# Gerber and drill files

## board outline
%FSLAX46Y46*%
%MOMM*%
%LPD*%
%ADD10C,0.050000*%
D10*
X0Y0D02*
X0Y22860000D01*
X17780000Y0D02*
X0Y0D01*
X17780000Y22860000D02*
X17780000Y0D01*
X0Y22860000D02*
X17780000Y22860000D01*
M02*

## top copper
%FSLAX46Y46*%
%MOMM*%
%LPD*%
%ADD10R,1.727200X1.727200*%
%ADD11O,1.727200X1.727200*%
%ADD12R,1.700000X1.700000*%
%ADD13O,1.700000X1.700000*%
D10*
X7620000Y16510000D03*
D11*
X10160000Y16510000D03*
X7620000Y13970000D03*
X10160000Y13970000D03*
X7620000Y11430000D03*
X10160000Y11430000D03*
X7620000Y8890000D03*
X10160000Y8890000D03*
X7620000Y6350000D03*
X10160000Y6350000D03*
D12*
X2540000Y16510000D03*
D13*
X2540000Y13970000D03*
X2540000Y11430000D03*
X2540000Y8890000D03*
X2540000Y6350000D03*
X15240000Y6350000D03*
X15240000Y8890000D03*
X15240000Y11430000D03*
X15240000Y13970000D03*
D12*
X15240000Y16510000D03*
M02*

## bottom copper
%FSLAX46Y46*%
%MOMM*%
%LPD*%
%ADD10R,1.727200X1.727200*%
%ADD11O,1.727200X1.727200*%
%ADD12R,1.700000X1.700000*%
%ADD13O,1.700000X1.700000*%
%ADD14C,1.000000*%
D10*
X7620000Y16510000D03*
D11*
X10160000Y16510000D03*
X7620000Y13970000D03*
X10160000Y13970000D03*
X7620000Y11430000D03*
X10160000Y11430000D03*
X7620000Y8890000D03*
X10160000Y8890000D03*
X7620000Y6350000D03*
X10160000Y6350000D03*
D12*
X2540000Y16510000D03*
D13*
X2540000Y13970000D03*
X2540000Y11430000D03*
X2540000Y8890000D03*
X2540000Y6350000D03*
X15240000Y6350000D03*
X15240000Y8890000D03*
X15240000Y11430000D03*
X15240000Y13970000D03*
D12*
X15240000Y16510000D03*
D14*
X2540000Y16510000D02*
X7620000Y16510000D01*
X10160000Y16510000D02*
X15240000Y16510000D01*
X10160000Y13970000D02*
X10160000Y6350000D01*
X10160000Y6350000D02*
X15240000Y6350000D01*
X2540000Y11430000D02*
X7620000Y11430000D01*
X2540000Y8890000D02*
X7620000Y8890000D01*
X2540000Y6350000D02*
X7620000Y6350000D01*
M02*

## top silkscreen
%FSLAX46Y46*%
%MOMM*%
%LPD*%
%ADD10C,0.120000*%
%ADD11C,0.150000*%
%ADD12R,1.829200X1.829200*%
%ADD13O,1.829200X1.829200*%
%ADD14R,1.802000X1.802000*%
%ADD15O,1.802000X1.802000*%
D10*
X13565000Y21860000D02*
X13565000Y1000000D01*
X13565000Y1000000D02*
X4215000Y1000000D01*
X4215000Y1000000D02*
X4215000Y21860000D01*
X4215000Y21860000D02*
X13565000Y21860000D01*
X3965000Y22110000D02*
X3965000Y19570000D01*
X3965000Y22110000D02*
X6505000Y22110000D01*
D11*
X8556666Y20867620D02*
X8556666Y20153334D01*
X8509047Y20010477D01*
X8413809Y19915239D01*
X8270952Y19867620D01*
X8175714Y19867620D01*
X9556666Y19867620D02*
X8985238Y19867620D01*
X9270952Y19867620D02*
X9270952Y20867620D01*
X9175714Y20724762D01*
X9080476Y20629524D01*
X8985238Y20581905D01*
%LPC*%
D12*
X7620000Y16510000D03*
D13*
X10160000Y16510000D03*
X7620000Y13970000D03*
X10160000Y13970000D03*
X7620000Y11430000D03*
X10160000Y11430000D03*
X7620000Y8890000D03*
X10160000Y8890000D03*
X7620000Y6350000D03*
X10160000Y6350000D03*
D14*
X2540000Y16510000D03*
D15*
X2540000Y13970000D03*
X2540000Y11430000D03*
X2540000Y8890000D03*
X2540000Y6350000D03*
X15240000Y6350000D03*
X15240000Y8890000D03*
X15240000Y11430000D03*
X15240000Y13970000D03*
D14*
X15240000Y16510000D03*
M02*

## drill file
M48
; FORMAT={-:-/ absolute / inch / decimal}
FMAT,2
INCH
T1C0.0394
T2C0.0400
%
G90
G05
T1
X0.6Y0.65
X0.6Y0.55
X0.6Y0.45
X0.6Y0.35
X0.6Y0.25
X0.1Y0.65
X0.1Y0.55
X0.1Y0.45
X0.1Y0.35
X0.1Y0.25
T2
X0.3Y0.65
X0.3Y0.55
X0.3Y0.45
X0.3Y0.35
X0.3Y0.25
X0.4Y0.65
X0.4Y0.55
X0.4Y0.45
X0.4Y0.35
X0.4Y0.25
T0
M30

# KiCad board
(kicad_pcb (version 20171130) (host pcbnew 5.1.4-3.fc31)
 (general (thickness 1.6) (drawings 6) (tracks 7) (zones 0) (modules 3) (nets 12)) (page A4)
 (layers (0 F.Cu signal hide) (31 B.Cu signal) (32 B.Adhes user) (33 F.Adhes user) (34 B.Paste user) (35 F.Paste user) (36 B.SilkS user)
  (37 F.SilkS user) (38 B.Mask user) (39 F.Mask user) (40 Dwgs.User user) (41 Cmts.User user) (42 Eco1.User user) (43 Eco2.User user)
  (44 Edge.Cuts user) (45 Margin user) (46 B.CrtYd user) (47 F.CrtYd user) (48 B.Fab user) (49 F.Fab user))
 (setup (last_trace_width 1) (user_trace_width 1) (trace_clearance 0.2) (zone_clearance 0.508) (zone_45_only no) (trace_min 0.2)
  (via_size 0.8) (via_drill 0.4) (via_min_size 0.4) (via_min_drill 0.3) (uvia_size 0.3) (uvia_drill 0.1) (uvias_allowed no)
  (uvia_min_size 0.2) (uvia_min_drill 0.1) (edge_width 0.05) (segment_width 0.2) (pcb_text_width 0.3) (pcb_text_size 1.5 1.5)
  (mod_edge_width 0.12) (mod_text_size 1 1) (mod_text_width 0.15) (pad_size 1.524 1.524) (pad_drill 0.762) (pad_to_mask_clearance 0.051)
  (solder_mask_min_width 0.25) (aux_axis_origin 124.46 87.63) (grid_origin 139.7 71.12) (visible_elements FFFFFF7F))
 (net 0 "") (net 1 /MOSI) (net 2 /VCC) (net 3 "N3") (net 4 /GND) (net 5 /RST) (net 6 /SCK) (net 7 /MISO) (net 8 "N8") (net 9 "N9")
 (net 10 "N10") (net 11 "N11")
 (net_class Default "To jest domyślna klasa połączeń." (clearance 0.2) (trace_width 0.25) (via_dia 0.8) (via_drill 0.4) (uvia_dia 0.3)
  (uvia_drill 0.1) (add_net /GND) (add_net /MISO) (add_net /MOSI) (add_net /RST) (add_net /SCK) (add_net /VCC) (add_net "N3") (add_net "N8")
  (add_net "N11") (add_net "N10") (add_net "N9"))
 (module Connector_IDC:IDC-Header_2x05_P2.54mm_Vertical (layer F.Cu) (at 132.08 71.12)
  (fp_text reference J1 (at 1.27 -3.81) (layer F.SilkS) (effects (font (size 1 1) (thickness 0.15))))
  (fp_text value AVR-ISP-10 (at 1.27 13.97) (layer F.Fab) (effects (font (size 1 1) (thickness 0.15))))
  (fp_line (start 5.945 -5.35) (end 5.945 15.51) (layer F.SilkS) (width 0.12))
  (fp_line (start 5.945 15.51) (end -3.405 15.51) (layer F.SilkS) (width 0.12))
  (fp_line (start -3.405 15.51) (end -3.405 -5.35) (layer F.SilkS) (width 0.12))
  (fp_line (start -3.405 -5.35) (end 5.945 -5.35) (layer F.SilkS) (width 0.12))
  (fp_line (start -3.655 -5.6) (end -3.655 -3.06) (layer F.SilkS) (width 0.12))
  (fp_line (start -3.655 -5.6) (end -1.115 -5.6) (layer F.SilkS) (width 0.12))
  (pad 1 thru_hole rect (at 0 0) (size 1.7272 1.7272) (drill 1.016) (layers *.Cu *.Mask) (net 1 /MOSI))
  (pad 2 thru_hole oval (at 2.54 0) (size 1.7272 1.7272) (drill 1.016) (layers *.Cu *.Mask) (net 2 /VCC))
  (pad 3 thru_hole oval (at 0 2.54) (size 1.7272 1.7272) (drill 1.016) (layers *.Cu *.Mask) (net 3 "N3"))
  (pad 4 thru_hole oval (at 2.54 2.54) (size 1.7272 1.7272) (drill 1.016) (layers *.Cu *.Mask) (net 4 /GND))
  (pad 5 thru_hole oval (at 0 5.08) (size 1.7272 1.7272) (drill 1.016) (layers *.Cu *.Mask) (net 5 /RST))
  (pad 6 thru_hole oval (at 2.54 5.08) (size 1.7272 1.7272) (drill 1.016) (layers *.Cu *.Mask) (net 4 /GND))
  (pad 7 thru_hole oval (at 0 7.62) (size 1.7272 1.7272) (drill 1.016) (layers *.Cu *.Mask) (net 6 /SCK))
  (pad 8 thru_hole oval (at 2.54 7.62) (size 1.7272 1.7272) (drill 1.016) (layers *.Cu *.Mask) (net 4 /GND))
  (pad 9 thru_hole oval (at 0 10.16) (size 1.7272 1.7272) (drill 1.016) (layers *.Cu *.Mask) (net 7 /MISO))
  (pad 10 thru_hole oval (at 2.54 10.16) (size 1.7272 1.7272) (drill 1.016) (layers *.Cu *.Mask) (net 4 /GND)))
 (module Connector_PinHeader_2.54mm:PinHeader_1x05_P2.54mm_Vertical (layer B.Cu) (at 127 71.12 180)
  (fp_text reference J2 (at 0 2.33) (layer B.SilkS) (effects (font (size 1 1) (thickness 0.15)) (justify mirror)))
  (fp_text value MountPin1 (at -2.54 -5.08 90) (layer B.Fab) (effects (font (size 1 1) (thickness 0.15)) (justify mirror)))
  (pad 1 thru_hole rect (at 0 0 180) (size 1.7 1.7) (drill 1) (layers *.Cu *.Mask) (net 1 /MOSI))
  (pad 2 thru_hole oval (at 0 -2.54 180) (size 1.7 1.7) (drill 1) (layers *.Cu *.Mask) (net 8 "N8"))
  (pad 3 thru_hole oval (at 0 -5.08 180) (size 1.7 1.7) (drill 1) (layers *.Cu *.Mask) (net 5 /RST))
  (pad 4 thru_hole oval (at 0 -7.62 180) (size 1.7 1.7) (drill 1) (layers *.Cu *.Mask) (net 6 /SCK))
  (pad 5 thru_hole oval (at 0 -10.16 180) (size 1.7 1.7) (drill 1) (layers *.Cu *.Mask) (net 7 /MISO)))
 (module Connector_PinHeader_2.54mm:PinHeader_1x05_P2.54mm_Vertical (layer B.Cu) (at 139.7 71.12 180)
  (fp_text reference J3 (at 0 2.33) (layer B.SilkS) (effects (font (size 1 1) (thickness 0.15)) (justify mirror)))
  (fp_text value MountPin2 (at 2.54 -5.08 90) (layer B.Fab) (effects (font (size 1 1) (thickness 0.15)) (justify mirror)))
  (pad 5 thru_hole oval (at 0 -10.16 180) (size 1.7 1.7) (drill 1) (layers *.Cu *.Mask) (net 4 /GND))
  (pad 4 thru_hole oval (at 0 -7.62 180) (size 1.7 1.7) (drill 1) (layers *.Cu *.Mask) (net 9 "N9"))
  (pad 3 thru_hole oval (at 0 -5.08 180) (size 1.7 1.7) (drill 1) (layers *.Cu *.Mask) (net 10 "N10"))
  (pad 2 thru_hole oval (at 0 -2.54 180) (size 1.7 1.7) (drill 1) (layers *.Cu *.Mask) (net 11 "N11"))
  (pad 1 thru_hole rect (at 0 0 180) (size 1.7 1.7) (drill 1) (layers *.Cu *.Mask) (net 2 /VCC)))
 (gr_line (start 124.46 87.63) (end 124.46 64.77) (layer Edge.Cuts) (width 0.05))
 (gr_line (start 142.24 87.63) (end 124.46 87.63) (layer Edge.Cuts) (width 0.05))
 (gr_line (start 142.24 64.77) (end 142.24 87.63) (layer Edge.Cuts) (width 0.05))
 (gr_line (start 124.46 64.77) (end 142.24 64.77) (layer Edge.Cuts) (width 0.05))
 (segment (start 127 71.12) (end 132.08 71.12) (width 1) (layer B.Cu) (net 1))
 (segment (start 134.62 71.12) (end 139.7 71.12) (width 1) (layer B.Cu) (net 2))
 (segment (start 134.62 73.66) (end 134.62 81.28) (width 1) (layer B.Cu) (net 4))
 (segment (start 134.62 81.28) (end 139.7 81.28) (width 1) (layer B.Cu) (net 4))
 (segment (start 127 76.2) (end 132.08 76.2) (width 1) (layer B.Cu) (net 5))
 (segment (start 127 78.74) (end 132.08 78.74) (width 1) (layer B.Cu) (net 6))
 (segment (start 127 81.28) (end 132.08 81.28) (width 1) (layer B.Cu) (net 7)))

